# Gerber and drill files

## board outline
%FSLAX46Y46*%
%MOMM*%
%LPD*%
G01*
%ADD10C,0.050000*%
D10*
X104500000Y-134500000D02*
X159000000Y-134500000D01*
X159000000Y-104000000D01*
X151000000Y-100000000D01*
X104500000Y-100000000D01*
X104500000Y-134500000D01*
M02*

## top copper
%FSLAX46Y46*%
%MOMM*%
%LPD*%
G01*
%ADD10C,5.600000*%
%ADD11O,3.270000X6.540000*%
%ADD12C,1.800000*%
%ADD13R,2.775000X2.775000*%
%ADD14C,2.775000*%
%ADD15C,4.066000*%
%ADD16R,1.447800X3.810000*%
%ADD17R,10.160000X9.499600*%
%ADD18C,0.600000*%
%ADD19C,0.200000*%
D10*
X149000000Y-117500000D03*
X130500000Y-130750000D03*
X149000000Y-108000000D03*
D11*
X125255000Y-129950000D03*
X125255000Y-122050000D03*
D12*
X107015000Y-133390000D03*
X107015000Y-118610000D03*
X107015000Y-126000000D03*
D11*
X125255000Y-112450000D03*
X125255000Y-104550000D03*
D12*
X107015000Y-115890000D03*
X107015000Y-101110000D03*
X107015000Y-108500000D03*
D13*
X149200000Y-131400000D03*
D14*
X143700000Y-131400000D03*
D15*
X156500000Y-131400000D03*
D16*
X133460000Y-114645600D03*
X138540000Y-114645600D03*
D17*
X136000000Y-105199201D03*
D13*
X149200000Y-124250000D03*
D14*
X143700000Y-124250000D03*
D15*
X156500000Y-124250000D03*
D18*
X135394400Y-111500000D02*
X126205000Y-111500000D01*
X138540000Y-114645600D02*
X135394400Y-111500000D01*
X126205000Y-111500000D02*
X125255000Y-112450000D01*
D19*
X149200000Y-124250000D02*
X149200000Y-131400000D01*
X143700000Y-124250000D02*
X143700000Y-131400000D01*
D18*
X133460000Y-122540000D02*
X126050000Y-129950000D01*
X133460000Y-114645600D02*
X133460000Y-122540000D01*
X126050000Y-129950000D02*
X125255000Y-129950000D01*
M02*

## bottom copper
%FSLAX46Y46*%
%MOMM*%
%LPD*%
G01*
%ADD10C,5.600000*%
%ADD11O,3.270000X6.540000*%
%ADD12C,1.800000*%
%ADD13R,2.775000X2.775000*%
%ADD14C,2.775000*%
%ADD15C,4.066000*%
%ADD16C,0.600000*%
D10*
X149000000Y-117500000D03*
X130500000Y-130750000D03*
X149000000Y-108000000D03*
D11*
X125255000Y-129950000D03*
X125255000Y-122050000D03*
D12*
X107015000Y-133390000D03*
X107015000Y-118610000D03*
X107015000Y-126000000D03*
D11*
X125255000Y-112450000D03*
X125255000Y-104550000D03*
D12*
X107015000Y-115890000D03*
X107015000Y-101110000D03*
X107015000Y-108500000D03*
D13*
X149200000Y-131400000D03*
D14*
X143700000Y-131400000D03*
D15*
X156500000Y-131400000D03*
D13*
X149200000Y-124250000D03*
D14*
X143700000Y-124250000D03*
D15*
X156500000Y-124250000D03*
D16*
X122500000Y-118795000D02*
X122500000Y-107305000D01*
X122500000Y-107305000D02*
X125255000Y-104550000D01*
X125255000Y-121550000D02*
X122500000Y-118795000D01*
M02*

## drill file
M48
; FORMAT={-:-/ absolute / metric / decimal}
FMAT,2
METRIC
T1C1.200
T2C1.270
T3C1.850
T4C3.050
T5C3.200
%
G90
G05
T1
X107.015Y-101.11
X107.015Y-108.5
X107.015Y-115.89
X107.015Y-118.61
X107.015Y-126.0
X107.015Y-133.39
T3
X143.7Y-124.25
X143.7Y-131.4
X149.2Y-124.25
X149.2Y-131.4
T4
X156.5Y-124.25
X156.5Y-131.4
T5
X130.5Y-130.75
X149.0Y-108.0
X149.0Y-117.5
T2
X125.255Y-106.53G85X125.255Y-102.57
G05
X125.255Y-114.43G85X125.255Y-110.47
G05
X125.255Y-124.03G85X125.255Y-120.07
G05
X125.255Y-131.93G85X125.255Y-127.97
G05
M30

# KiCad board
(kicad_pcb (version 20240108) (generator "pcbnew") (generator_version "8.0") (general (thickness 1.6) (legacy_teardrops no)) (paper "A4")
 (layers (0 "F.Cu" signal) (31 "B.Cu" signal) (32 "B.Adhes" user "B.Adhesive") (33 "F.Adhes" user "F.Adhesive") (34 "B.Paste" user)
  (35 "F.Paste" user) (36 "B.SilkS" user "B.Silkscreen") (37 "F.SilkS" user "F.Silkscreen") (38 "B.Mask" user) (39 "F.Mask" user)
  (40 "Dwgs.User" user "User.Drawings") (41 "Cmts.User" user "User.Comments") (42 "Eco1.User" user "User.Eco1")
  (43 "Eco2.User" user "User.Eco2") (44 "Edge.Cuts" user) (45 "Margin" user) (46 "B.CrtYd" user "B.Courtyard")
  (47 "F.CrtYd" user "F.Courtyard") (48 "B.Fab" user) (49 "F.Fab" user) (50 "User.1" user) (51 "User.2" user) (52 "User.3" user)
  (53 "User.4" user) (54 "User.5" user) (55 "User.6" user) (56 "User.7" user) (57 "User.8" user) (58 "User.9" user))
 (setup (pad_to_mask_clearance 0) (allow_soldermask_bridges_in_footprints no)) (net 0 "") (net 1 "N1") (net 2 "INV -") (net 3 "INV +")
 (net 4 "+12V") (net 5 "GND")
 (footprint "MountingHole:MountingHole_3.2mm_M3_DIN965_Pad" (layer "F.Cu") (at 149 117.5)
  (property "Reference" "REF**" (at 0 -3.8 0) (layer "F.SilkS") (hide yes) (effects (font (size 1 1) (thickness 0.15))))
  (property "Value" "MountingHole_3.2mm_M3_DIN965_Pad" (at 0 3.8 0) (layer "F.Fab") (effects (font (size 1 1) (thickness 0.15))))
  (pad "1" thru_hole circle (at 0 0) (size 5.6 5.6) (drill 3.2) (layers "*.Cu" "*.Mask") (remove_unused_layers no)))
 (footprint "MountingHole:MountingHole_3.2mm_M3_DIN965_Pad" (layer "F.Cu") (at 130.5 130.75)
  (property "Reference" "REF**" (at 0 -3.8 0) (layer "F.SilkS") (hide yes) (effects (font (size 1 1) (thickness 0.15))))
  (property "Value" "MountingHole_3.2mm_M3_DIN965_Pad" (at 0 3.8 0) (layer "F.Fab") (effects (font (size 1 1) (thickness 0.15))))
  (pad "1" thru_hole circle (at 0 0) (size 5.6 5.6) (drill 3.2) (layers "*.Cu" "*.Mask") (remove_unused_layers no)))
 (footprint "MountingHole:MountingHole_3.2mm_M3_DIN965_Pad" (layer "F.Cu") (at 149 108)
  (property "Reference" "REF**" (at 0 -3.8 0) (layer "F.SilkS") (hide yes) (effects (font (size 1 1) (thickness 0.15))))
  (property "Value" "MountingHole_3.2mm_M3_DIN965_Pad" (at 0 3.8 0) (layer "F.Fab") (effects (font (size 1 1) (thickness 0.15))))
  (pad "1" thru_hole circle (at 0 0) (size 5.6 5.6) (drill 3.2) (layers "*.Cu" "*.Mask") (remove_unused_layers no)))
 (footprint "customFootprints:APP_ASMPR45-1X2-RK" (layer "F.Cu") (at 107.015 126 90)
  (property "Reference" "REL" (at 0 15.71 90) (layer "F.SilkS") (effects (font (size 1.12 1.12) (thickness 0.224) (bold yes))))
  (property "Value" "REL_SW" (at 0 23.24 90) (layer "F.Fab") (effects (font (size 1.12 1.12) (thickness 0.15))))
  (pad "1" thru_hole oval (at -3.95 18.24 90) (size 6.54 3.27) (drill oval 5.23 1.27) (layers "*.Cu" "*.Mask") (remove_unused_layers no)
   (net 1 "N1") (solder_mask_margin 0.102))
  (pad "2" thru_hole oval (at 3.95 18.24 90) (size 6.54 3.27) (drill oval 5.23 1.27) (layers "*.Cu" "*.Mask") (remove_unused_layers no)
   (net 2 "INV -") (solder_mask_margin 0.102))
  (pad "P3" thru_hole circle (at -7.39 0 90) (size 1.8 1.8) (drill 1.2) (layers "*.Cu" "*.Mask") (remove_unused_layers no)
   (solder_mask_margin 0.102))
  (pad "P4" thru_hole circle (at 7.39 0 90) (size 1.8 1.8) (drill 1.2) (layers "*.Cu" "*.Mask") (remove_unused_layers no)
   (solder_mask_margin 0.102))
  (pad "P5" thru_hole circle (at 0 0 90) (size 1.8 1.8) (drill 1.2) (layers "*.Cu" "*.Mask") (remove_unused_layers no)
   (solder_mask_margin 0.102)))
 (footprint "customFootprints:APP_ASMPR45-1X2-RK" (layer "F.Cu") (at 107.015 108.5 90)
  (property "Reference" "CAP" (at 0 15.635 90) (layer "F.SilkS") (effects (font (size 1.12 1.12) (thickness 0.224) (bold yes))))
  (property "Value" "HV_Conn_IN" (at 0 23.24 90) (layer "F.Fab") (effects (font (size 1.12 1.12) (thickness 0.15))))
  (pad "1" thru_hole oval (at -3.95 18.24 90) (size 6.54 3.27) (drill oval 5.23 1.27) (layers "*.Cu" "*.Mask") (remove_unused_layers no)
   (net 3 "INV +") (solder_mask_margin 0.102))
  (pad "2" thru_hole oval (at 3.95 18.24 90) (size 6.54 3.27) (drill oval 5.23 1.27) (layers "*.Cu" "*.Mask") (remove_unused_layers no)
   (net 2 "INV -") (solder_mask_margin 0.102))
  (pad "P3" thru_hole circle (at -7.39 0 90) (size 1.8 1.8) (drill 1.2) (layers "*.Cu" "*.Mask") (remove_unused_layers no)
   (solder_mask_margin 0.102))
  (pad "P4" thru_hole circle (at 7.39 0 90) (size 1.8 1.8) (drill 1.2) (layers "*.Cu" "*.Mask") (remove_unused_layers no)
   (solder_mask_margin 0.102))
  (pad "P5" thru_hole circle (at 0 0 90) (size 1.8 1.8) (drill 1.2) (layers "*.Cu" "*.Mask") (remove_unused_layers no)
   (solder_mask_margin 0.102)))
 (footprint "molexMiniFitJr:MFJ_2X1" (layer "F.Cu") (at 149.2 131.4 90)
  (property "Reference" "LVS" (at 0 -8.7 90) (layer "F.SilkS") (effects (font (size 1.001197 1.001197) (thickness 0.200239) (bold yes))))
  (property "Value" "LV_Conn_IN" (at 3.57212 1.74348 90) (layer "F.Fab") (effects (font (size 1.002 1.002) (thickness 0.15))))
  (pad "1" thru_hole rect (at 0 0 90) (size 2.775 2.775) (drill 1.85) (layers "*.Cu" "*.Mask") (remove_unused_layers no) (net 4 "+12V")
   (solder_mask_margin 0.0762))
  (pad "2" thru_hole circle (at 0 -5.5 90) (size 2.775 2.775) (drill 1.85) (layers "*.Cu" "*.Mask") (remove_unused_layers no) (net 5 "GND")
   (solder_mask_margin 0.0762))
  (pad "P$3" thru_hole circle (at 0 7.3 90) (size 4.066 4.066) (drill 3.05) (layers "*.Cu" "*.Mask") (remove_unused_layers no)
   (solder_mask_margin 0.0762)))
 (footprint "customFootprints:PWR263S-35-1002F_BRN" (layer "F.Cu") (at 136 105.199201)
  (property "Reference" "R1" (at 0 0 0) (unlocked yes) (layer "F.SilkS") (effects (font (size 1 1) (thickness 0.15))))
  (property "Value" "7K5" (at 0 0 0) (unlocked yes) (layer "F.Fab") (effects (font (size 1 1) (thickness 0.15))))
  (pad "1" smd rect (at -2.54 9.446399) (size 1.4478 3.81) (layers "F.Cu" "F.Paste" "F.Mask") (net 1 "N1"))
  (pad "2" smd rect (at 2.54 9.446399) (size 1.4478 3.81) (layers "F.Cu" "F.Paste" "F.Mask") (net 3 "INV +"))
  (pad "3" smd rect (at 0 0) (size 10.16 9.4996) (layers "F.Cu" "F.Paste" "F.Mask")))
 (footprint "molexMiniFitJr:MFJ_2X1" (layer "F.Cu") (at 149.2 124.25 90)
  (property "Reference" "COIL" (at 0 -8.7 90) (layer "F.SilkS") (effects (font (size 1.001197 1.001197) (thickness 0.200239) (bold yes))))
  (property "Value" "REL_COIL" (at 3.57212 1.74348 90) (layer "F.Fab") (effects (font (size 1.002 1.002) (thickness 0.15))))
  (pad "1" thru_hole rect (at 0 0 90) (size 2.775 2.775) (drill 1.85) (layers "*.Cu" "*.Mask") (remove_unused_layers no) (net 4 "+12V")
   (solder_mask_margin 0.0762))
  (pad "2" thru_hole circle (at 0 -5.5 90) (size 2.775 2.775) (drill 1.85) (layers "*.Cu" "*.Mask") (remove_unused_layers no) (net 5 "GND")
   (solder_mask_margin 0.0762))
  (pad "P$3" thru_hole circle (at 0 7.3 90) (size 4.066 4.066) (drill 3.05) (layers "*.Cu" "*.Mask") (remove_unused_layers no)
   (solder_mask_margin 0.0762)))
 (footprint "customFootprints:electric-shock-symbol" (layer "F.Cu") (at 130.5 124 90)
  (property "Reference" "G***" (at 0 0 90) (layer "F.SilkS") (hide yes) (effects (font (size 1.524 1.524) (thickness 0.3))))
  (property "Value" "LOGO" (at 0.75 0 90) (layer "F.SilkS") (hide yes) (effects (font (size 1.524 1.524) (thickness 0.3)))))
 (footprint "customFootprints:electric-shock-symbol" (layer "B.Cu") (at 130.5 124 -90)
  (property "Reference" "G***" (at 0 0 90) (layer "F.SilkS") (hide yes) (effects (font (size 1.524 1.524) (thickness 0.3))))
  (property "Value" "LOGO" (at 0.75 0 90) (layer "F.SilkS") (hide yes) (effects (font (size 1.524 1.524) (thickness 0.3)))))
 (gr_poly
  (pts (xy 104.5 134.5) (xy 159 134.5) (xy 159 104) (xy 151 100) (xy 104.5 100)) (stroke (width 0.05) (type solid)) (fill none)
  (layer "Edge.Cuts"))
 (segment (start 135.3944 111.5) (end 126.205 111.5) (width 0.6) (layer "F.Cu") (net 3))
 (segment (start 138.54 114.6456) (end 135.3944 111.5) (width 0.6) (layer "F.Cu") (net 3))
 (segment (start 126.205 111.5) (end 125.255 112.45) (width 0.6) (layer "F.Cu") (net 3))
 (segment (start 149.2 124.25) (end 149.2 131.4) (width 0.2) (layer "F.Cu") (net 4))
 (segment (start 122.5 118.795) (end 122.5 107.305) (width 0.6) (layer "B.Cu") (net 2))
 (segment (start 122.5 107.305) (end 125.255 104.55) (width 0.6) (layer "B.Cu") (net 2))
 (segment (start 125.255 121.55) (end 122.5 118.795) (width 0.6) (layer "B.Cu") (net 2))
 (segment (start 143.7 124.25) (end 143.7 131.4) (width 0.2) (layer "F.Cu") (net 5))
 (segment (start 133.46 122.54) (end 126.05 129.95) (width 0.6) (layer "F.Cu") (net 1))
 (segment (start 133.46 114.6456) (end 133.46 122.54) (width 0.6) (layer "F.Cu") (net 1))
 (segment (start 126.05 129.95) (end 125.255 129.95) (width 0.6) (layer "F.Cu") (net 1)))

